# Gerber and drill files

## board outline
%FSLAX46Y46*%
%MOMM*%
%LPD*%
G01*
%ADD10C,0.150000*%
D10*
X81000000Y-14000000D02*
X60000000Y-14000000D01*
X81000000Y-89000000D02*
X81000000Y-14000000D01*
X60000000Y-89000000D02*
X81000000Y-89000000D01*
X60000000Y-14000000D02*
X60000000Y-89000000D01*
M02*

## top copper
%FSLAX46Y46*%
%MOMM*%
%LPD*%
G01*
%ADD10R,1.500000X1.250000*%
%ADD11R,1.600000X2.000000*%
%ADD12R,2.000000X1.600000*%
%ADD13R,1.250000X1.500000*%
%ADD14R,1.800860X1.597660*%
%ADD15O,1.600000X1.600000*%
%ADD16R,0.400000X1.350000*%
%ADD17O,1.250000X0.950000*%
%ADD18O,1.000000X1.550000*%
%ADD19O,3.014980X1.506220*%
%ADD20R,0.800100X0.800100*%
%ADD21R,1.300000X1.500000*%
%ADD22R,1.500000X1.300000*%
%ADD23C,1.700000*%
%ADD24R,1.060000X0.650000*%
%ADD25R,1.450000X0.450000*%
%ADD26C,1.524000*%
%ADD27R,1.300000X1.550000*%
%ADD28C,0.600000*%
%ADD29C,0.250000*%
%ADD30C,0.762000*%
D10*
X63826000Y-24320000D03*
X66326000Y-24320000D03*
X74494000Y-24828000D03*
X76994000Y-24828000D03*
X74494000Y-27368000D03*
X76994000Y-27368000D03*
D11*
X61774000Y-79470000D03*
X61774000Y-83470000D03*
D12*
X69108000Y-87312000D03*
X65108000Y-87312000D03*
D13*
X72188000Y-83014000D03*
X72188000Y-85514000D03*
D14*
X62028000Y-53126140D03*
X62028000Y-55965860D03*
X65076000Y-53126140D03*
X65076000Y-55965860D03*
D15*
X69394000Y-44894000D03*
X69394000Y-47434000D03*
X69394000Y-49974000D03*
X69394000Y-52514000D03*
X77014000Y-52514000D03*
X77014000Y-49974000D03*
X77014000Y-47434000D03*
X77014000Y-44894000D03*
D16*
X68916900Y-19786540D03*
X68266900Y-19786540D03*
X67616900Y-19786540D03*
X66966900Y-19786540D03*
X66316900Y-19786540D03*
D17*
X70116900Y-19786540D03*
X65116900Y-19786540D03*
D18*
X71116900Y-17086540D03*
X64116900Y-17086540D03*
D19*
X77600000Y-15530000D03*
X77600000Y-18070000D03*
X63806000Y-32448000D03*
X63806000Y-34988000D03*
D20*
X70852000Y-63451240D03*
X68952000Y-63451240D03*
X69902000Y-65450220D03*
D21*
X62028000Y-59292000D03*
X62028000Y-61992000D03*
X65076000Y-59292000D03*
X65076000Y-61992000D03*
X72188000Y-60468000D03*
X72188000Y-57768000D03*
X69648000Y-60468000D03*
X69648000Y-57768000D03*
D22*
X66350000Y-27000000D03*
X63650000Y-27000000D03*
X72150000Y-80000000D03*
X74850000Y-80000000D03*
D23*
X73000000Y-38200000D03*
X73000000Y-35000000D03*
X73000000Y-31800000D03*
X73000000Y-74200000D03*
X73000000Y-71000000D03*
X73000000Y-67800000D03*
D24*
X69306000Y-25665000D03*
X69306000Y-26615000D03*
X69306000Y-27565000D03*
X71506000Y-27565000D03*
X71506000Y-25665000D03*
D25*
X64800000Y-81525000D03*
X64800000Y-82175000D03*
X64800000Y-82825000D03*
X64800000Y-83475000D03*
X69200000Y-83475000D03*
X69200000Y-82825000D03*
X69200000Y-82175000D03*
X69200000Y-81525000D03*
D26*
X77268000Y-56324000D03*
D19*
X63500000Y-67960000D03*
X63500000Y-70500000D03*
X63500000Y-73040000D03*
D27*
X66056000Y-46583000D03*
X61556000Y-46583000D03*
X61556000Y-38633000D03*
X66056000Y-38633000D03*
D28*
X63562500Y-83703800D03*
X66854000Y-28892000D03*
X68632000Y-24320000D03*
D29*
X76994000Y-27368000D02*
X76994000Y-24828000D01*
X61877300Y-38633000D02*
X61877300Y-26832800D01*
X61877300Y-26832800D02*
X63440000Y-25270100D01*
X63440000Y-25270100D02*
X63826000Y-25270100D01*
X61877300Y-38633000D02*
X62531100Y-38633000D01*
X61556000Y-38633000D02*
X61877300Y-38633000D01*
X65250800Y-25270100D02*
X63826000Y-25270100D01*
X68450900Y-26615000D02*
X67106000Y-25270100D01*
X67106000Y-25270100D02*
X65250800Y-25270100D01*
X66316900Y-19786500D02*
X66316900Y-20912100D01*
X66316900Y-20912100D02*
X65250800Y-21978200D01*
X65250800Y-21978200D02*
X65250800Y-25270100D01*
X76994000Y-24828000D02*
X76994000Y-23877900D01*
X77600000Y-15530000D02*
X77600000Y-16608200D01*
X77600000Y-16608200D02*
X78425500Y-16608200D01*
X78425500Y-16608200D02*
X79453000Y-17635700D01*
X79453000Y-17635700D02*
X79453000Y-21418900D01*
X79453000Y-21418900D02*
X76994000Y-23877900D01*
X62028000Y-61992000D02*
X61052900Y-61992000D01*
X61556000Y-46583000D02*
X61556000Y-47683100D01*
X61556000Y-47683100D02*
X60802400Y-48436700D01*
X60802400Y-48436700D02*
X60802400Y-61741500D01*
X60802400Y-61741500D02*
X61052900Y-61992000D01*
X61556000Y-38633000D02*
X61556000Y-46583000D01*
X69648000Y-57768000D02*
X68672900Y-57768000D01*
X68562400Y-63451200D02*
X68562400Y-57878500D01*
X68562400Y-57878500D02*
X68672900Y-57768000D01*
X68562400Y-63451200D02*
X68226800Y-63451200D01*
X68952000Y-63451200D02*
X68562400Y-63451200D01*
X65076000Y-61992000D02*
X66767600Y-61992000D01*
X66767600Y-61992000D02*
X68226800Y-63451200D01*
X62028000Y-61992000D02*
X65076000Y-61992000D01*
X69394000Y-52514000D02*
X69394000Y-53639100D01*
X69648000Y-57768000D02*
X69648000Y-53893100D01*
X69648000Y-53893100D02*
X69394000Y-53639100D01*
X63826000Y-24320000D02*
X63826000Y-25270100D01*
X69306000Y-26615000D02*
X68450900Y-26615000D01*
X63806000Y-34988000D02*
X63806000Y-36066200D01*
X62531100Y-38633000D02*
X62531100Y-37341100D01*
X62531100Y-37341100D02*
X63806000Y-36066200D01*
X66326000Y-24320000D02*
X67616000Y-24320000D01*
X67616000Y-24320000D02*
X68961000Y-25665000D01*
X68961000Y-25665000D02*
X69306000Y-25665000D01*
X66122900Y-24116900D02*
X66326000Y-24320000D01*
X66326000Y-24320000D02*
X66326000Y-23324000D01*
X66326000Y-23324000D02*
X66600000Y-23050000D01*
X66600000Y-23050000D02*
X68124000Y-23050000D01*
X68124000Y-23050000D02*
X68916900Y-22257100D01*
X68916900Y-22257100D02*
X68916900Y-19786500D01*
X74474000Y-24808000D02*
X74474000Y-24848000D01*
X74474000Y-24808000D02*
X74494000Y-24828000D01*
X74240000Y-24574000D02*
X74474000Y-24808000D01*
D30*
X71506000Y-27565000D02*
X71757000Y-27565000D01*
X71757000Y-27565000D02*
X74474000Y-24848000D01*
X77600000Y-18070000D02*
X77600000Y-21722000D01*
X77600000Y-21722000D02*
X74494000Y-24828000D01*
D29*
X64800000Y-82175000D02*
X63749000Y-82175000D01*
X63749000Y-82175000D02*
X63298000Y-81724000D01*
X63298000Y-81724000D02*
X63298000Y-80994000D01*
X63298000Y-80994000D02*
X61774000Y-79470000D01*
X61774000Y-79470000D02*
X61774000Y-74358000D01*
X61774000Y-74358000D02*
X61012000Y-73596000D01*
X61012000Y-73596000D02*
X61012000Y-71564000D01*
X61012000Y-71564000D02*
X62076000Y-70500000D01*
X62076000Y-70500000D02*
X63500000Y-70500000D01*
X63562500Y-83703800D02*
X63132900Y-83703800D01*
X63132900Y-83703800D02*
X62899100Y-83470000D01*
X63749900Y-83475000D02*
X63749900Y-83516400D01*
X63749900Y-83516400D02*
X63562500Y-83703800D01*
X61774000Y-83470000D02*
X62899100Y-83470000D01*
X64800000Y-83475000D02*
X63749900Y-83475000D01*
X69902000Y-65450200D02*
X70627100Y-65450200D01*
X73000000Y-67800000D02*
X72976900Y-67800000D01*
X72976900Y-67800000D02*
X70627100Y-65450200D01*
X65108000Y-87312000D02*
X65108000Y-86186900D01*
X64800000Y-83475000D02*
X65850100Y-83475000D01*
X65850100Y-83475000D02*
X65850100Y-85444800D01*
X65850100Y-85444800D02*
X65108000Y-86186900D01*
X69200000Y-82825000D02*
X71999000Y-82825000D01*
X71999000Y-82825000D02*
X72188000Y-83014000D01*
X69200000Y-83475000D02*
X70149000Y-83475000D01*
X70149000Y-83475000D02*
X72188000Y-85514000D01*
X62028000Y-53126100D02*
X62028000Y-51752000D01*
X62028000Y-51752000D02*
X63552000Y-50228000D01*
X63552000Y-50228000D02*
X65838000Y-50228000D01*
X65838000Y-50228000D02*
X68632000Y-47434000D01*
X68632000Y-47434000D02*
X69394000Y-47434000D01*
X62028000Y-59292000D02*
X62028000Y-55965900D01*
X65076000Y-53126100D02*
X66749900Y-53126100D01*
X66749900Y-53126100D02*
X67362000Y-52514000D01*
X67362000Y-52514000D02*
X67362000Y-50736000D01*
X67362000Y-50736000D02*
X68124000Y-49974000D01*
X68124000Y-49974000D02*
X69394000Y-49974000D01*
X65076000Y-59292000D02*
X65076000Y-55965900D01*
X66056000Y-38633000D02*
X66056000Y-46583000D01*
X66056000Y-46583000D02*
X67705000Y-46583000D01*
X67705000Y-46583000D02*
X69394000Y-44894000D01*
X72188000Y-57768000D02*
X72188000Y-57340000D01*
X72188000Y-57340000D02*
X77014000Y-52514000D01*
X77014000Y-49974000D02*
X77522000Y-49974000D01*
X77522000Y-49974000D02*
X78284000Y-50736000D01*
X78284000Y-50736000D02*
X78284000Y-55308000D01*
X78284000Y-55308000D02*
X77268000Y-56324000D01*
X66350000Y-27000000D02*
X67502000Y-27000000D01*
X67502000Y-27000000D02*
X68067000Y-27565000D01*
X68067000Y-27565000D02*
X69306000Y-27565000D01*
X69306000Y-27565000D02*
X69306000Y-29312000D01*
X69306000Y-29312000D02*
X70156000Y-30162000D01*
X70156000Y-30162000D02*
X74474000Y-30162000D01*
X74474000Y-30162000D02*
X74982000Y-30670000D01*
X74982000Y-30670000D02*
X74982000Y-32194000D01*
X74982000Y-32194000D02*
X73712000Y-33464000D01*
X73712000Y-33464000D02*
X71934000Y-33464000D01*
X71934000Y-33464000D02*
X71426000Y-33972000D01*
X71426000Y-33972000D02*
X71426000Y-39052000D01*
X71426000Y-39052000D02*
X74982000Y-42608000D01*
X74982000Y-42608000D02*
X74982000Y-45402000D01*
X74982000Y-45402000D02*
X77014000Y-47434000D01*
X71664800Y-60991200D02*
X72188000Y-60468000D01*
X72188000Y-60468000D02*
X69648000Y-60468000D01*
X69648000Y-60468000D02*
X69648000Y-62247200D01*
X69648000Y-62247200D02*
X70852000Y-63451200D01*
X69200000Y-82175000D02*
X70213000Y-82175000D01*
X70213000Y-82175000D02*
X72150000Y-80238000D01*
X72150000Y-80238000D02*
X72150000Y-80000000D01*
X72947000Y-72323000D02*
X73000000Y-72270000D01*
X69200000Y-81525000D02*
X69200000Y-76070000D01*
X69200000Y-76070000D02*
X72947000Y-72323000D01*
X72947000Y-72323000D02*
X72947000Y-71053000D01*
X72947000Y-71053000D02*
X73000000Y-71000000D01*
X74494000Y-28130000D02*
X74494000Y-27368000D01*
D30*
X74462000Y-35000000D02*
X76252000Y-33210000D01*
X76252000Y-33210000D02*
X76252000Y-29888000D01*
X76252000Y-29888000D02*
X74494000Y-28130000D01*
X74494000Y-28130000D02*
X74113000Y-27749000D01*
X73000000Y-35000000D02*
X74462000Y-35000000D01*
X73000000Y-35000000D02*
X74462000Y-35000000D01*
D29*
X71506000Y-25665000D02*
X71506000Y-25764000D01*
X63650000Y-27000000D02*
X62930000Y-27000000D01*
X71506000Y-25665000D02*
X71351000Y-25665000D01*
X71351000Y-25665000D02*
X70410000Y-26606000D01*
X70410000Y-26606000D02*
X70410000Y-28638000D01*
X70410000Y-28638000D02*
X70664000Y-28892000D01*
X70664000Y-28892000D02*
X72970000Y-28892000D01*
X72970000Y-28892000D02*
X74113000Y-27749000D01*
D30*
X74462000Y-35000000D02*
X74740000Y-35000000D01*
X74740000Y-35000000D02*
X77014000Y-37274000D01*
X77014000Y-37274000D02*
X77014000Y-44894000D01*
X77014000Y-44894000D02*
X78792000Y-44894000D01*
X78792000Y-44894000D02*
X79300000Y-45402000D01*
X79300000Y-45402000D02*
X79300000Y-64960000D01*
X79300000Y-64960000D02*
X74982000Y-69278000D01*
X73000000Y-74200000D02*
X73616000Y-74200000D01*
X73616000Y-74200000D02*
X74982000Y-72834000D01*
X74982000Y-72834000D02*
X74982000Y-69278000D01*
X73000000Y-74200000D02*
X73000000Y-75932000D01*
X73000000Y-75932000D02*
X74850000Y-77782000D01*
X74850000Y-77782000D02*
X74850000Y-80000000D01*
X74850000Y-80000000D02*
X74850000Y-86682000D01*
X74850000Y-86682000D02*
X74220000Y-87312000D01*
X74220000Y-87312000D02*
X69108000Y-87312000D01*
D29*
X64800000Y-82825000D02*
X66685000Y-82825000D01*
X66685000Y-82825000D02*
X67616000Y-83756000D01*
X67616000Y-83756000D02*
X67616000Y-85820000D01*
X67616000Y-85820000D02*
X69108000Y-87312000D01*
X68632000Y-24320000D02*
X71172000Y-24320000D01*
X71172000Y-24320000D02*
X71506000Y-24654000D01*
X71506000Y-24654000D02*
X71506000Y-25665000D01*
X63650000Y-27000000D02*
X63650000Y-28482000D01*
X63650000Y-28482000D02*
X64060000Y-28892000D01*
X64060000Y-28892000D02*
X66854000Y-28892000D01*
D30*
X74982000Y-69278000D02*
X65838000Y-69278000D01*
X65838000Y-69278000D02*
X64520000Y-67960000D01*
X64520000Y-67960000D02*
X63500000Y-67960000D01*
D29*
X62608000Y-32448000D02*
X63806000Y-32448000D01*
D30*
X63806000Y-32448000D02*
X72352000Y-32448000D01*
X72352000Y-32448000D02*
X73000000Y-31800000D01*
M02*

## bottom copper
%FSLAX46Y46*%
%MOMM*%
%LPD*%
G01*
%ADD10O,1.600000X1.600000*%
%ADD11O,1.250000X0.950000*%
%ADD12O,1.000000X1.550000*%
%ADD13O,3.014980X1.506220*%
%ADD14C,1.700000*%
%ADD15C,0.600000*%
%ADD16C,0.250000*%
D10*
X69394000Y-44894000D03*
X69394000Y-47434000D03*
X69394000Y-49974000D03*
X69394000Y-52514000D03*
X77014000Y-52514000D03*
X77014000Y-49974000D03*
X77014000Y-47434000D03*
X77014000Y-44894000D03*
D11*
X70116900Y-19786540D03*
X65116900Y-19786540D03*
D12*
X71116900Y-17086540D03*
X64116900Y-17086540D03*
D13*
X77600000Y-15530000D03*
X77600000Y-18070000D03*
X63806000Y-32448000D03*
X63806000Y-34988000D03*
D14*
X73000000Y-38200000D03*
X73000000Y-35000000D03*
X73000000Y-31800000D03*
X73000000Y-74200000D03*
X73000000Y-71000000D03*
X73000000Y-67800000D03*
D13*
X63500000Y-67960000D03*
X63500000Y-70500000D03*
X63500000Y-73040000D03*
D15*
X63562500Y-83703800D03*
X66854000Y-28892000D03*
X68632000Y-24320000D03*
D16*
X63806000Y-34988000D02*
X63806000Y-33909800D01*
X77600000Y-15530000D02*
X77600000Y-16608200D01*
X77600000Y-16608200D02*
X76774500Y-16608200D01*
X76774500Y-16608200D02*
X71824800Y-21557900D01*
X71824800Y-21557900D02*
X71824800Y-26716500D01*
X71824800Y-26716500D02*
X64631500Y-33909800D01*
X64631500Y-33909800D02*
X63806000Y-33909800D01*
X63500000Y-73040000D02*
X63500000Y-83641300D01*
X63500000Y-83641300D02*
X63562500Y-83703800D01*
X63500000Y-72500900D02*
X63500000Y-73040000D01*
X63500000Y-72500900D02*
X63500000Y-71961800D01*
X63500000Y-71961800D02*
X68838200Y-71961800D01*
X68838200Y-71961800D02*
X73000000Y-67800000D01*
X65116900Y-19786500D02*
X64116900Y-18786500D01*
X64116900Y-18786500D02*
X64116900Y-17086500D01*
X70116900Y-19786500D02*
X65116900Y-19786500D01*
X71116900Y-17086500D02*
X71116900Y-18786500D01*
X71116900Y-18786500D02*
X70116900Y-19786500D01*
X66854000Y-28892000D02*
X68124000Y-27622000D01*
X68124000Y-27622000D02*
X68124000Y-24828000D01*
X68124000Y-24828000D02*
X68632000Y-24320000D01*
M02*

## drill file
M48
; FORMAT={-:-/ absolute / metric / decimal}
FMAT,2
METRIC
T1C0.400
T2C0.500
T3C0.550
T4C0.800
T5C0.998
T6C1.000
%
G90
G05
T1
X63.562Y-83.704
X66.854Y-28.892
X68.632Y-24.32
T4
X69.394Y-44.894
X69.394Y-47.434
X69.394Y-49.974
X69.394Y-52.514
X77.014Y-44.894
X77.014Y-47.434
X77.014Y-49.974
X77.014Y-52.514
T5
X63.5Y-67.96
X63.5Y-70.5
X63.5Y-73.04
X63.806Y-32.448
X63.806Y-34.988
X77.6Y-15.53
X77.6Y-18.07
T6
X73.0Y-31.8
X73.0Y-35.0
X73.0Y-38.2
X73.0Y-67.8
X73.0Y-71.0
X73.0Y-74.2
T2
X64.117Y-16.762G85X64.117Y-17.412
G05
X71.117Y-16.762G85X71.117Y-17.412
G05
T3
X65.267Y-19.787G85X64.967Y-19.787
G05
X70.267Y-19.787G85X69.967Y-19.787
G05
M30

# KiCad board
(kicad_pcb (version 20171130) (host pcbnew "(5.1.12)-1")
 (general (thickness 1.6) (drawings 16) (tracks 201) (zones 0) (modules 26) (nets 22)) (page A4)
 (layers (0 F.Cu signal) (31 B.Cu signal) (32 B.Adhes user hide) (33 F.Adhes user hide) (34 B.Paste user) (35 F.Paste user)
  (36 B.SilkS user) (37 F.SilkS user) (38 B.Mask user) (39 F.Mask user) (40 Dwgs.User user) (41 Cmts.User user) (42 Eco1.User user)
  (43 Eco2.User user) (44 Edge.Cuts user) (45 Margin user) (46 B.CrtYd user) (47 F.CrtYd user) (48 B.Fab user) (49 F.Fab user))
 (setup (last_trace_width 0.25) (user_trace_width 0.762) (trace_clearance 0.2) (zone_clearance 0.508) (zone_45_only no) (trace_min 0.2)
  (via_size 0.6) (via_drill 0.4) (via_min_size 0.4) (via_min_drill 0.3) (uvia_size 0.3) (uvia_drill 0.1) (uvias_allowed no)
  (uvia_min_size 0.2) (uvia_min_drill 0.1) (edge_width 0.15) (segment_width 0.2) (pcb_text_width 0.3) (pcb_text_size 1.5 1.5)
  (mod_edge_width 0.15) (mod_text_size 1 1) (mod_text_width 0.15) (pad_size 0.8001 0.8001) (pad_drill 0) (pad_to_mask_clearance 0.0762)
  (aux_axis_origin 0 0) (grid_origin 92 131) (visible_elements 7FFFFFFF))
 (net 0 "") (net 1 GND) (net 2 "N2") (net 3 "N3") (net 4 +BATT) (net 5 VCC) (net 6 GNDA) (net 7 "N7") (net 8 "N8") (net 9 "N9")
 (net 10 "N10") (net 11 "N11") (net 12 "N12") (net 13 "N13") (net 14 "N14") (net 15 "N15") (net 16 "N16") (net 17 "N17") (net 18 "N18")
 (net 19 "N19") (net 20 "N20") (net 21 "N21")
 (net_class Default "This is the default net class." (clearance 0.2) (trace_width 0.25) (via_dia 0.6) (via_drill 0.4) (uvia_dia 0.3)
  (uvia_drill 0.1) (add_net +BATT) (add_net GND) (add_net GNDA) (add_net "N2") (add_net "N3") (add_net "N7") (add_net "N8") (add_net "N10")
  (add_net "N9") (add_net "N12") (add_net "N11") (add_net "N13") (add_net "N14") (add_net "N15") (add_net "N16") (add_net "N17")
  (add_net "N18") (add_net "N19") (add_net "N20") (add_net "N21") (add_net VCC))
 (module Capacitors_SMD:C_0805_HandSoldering (layer F.Cu) (at 65.076 24.32)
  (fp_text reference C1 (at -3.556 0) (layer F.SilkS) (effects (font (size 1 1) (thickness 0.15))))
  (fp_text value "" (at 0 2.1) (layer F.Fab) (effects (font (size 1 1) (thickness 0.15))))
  (pad 1 smd rect (at -1.25 0) (size 1.5 1.25) (layers F.Cu F.Paste F.Mask) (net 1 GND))
  (pad 2 smd rect (at 1.25 0) (size 1.5 1.25) (layers F.Cu F.Paste F.Mask) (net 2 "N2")))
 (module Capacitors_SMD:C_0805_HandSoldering (layer F.Cu) (at 75.744 24.828)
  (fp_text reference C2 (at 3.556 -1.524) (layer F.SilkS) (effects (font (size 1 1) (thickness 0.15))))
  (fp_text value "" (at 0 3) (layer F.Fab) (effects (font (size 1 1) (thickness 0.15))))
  (pad 1 smd rect (at -1.25 0) (size 1.5 1.25) (layers F.Cu F.Paste F.Mask) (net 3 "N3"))
  (pad 2 smd rect (at 1.25 0) (size 1.5 1.25) (layers F.Cu F.Paste F.Mask) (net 1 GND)))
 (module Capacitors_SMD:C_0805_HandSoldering (layer F.Cu) (at 75.744 27.368)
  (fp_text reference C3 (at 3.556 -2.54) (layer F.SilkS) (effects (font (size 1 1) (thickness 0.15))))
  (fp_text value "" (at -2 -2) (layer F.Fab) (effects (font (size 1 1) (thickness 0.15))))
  (pad 1 smd rect (at -1.25 0) (size 1.5 1.25) (layers F.Cu F.Paste F.Mask) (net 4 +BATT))
  (pad 2 smd rect (at 1.25 0) (size 1.5 1.25) (layers F.Cu F.Paste F.Mask) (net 1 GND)))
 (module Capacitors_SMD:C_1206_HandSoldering (layer F.Cu) (at 61.774 81.47 270)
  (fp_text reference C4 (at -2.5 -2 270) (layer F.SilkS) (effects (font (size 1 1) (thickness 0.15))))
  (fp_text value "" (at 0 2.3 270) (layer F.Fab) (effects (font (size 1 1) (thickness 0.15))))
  (pad 1 smd rect (at -2 0 270) (size 2 1.6) (layers F.Cu F.Paste F.Mask) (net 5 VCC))
  (pad 2 smd rect (at 2 0 270) (size 2 1.6) (layers F.Cu F.Paste F.Mask) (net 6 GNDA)))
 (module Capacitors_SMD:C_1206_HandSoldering (layer F.Cu) (at 67.108 87.312 180)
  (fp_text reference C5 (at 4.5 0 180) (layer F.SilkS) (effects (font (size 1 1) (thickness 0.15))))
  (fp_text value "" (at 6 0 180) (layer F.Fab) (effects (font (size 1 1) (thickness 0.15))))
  (pad 1 smd rect (at -2 0 180) (size 2 1.6) (layers F.Cu F.Paste F.Mask) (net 4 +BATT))
  (pad 2 smd rect (at 2 0 180) (size 2 1.6) (layers F.Cu F.Paste F.Mask) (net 6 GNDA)))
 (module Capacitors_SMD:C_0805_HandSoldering (layer F.Cu) (at 72.188 84.264 270)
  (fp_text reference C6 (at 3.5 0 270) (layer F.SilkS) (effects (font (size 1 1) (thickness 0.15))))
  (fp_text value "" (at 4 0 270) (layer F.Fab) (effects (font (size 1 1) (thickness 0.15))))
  (pad 1 smd rect (at -1.25 0 270) (size 1.5 1.25) (layers F.Cu F.Paste F.Mask) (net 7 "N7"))
  (pad 2 smd rect (at 1.25 0 270) (size 1.5 1.25) (layers F.Cu F.Paste F.Mask) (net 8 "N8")))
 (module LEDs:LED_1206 (layer F.Cu) (at 62.028 54.546 90)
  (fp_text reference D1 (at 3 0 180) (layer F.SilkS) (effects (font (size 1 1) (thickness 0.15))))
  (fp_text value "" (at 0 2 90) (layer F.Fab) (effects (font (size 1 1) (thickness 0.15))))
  (pad 2 smd rect (at 1.41986 0 270) (size 1.59766 1.80086) (layers F.Cu F.Paste F.Mask) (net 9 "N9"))
  (pad 1 smd rect (at -1.41986 0 270) (size 1.59766 1.80086) (layers F.Cu F.Paste F.Mask) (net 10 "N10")))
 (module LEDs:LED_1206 (layer F.Cu) (at 65.076 54.546 90)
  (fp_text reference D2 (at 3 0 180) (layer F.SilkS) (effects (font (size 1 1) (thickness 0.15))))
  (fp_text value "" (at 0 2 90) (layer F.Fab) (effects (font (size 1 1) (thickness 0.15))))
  (pad 2 smd rect (at 1.41986 0 270) (size 1.59766 1.80086) (layers F.Cu F.Paste F.Mask) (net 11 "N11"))
  (pad 1 smd rect (at -1.41986 0 270) (size 1.59766 1.80086) (layers F.Cu F.Paste F.Mask) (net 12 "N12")))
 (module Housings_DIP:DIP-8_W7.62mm (layer F.Cu) (at 69.394 44.894)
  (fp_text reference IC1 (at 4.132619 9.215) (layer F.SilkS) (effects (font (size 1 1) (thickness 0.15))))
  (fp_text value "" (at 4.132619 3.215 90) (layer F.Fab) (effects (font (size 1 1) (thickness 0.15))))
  (pad 1 thru_hole oval (at 0 0) (size 1.6 1.6) (drill 0.8) (layers *.Cu *.Mask F.SilkS) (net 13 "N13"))
  (pad 2 thru_hole oval (at 0 2.54) (size 1.6 1.6) (drill 0.8) (layers *.Cu *.Mask F.SilkS) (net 9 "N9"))
  (pad 3 thru_hole oval (at 0 5.08) (size 1.6 1.6) (drill 0.8) (layers *.Cu *.Mask F.SilkS) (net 11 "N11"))
  (pad 4 thru_hole oval (at 0 7.62) (size 1.6 1.6) (drill 0.8) (layers *.Cu *.Mask F.SilkS) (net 1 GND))
  (pad 5 thru_hole oval (at 7.62 7.62) (size 1.6 1.6) (drill 0.8) (layers *.Cu *.Mask F.SilkS) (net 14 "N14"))
  (pad 6 thru_hole oval (at 7.62 5.08) (size 1.6 1.6) (drill 0.8) (layers *.Cu *.Mask F.SilkS) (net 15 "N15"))
  (pad 7 thru_hole oval (at 7.62 2.54) (size 1.6 1.6) (drill 0.8) (layers *.Cu *.Mask F.SilkS) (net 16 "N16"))
  (pad 8 thru_hole oval (at 7.62 0) (size 1.6 1.6) (drill 0.8) (layers *.Cu *.Mask F.SilkS) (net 4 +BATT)))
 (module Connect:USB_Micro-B (layer F.Cu) (at 67.616 18.224 180)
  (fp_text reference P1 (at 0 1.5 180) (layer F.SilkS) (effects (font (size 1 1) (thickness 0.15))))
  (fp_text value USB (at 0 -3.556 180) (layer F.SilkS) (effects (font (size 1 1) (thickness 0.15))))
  (pad 1 smd rect (at -1.3009 -1.56254 270) (size 1.35 0.4) (layers F.Cu F.Paste F.Mask) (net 2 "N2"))
  (pad 2 smd rect (at -0.6509 -1.56254 270) (size 1.35 0.4) (layers F.Cu F.Paste F.Mask))
  (pad 3 smd rect (at -0.0009 -1.56254 270) (size 1.35 0.4) (layers F.Cu F.Paste F.Mask))
  (pad 4 smd rect (at 0.6491 -1.56254 270) (size 1.35 0.4) (layers F.Cu F.Paste F.Mask))
  (pad 5 smd rect (at 1.2991 -1.56254 270) (size 1.35 0.4) (layers F.Cu F.Paste F.Mask) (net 1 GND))
  (pad 6 thru_hole oval (at -2.5009 -1.56254 270) (size 0.95 1.25) (drill oval 0.55 0.85) (layers *.Cu *.Mask F.SilkS) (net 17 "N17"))
  (pad 6 thru_hole oval (at 2.4991 -1.56254 270) (size 0.95 1.25) (drill oval 0.55 0.85) (layers *.Cu *.Mask F.SilkS) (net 17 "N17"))
  (pad 6 thru_hole oval (at -3.5009 1.13746 270) (size 1.55 1) (drill oval 1.15 0.5) (layers *.Cu *.Mask F.SilkS) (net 17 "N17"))
  (pad 6 thru_hole oval (at 3.4991 1.13746 270) (size 1.55 1) (drill oval 1.15 0.5) (layers *.Cu *.Mask F.SilkS) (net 17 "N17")))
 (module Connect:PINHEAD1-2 (layer F.Cu) (at 77.6 16.8 270)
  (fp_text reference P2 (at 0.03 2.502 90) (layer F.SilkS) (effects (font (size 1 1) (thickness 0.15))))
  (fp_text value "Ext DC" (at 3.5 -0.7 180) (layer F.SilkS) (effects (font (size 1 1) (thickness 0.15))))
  (pad 1 thru_hole oval (at -1.27 0 270) (size 1.50622 3.01498) (drill 0.99822) (layers *.Cu *.Mask) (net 1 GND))
  (pad 2 thru_hole oval (at 1.27 0 270) (size 1.50622 3.01498) (drill 0.99822) (layers *.Cu *.Mask) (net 3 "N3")))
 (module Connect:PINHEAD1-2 (layer F.Cu) (at 63.806 33.718 270)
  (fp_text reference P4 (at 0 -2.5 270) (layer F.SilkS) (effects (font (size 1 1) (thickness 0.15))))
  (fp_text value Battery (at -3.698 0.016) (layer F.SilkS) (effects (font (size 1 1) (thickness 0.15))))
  (pad 1 thru_hole oval (at -1.27 0 270) (size 1.50622 3.01498) (drill 0.99822) (layers *.Cu *.Mask) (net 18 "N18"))
  (pad 2 thru_hole oval (at 1.27 0 270) (size 1.50622 3.01498) (drill 0.99822) (layers *.Cu *.Mask) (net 1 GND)))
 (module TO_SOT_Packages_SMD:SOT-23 (layer F.Cu) (at 69.902 64.452 180)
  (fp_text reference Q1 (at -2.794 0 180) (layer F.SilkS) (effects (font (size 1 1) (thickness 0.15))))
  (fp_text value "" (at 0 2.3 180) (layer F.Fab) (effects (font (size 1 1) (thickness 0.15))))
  (pad 2 smd rect (at -0.95 1.00076 180) (size 0.8001 0.8001) (layers F.Cu F.Paste F.Mask) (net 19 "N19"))
  (pad 3 smd rect (at 0.95 1.00076 180) (size 0.8001 0.8001) (layers F.Cu F.Paste F.Mask) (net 1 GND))
  (pad 1 smd rect (at 0 -0.99822 180) (size 0.8001 0.8001) (layers F.Cu F.Paste F.Mask) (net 6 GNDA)))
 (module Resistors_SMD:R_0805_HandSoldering (layer F.Cu) (at 62.028 60.642 270)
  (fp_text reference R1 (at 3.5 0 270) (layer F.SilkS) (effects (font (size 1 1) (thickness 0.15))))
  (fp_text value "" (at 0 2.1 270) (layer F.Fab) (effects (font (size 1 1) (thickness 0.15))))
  (pad 1 smd rect (at -1.35 0 270) (size 1.5 1.3) (layers F.Cu F.Paste F.Mask) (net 10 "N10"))
  (pad 2 smd rect (at 1.35 0 270) (size 1.5 1.3) (layers F.Cu F.Paste F.Mask) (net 1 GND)))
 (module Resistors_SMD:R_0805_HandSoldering (layer F.Cu) (at 65.076 60.642 270)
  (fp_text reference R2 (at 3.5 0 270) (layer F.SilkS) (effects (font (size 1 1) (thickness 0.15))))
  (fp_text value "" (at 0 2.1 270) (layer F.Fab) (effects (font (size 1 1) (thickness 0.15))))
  (pad 1 smd rect (at -1.35 0 270) (size 1.5 1.3) (layers F.Cu F.Paste F.Mask) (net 12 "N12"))
  (pad 2 smd rect (at 1.35 0 270) (size 1.5 1.3) (layers F.Cu F.Paste F.Mask) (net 1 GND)))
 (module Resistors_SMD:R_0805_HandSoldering (layer F.Cu) (at 72.188 59.118 90)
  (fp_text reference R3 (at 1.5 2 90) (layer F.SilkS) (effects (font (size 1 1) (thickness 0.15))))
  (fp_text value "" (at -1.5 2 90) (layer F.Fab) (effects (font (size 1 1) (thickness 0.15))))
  (pad 1 smd rect (at -1.35 0 90) (size 1.5 1.3) (layers F.Cu F.Paste F.Mask) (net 19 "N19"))
  (pad 2 smd rect (at 1.35 0 90) (size 1.5 1.3) (layers F.Cu F.Paste F.Mask) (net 14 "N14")))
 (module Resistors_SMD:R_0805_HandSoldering (layer F.Cu) (at 69.648 59.118 90)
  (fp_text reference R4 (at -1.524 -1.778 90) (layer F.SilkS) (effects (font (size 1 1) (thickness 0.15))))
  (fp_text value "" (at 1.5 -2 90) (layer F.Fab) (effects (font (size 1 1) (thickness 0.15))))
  (pad 1 smd rect (at -1.35 0 90) (size 1.5 1.3) (layers F.Cu F.Paste F.Mask) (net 19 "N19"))
  (pad 2 smd rect (at 1.35 0 90) (size 1.5 1.3) (layers F.Cu F.Paste F.Mask) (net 1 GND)))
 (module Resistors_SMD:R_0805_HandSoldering (layer F.Cu) (at 65 27 180)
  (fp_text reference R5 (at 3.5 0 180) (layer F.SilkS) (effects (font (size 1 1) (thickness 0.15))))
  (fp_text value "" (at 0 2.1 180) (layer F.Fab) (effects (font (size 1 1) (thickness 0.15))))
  (pad 1 smd rect (at -1.35 0 180) (size 1.5 1.3) (layers F.Cu F.Paste F.Mask) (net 16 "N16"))
  (pad 2 smd rect (at 1.35 0 180) (size 1.5 1.3) (layers F.Cu F.Paste F.Mask) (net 4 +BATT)))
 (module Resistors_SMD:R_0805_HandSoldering (layer F.Cu) (at 73.5 80)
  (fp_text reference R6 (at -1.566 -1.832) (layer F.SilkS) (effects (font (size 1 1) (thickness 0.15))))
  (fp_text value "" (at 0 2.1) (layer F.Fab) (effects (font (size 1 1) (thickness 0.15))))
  (pad 1 smd rect (at -1.35 0) (size 1.5 1.3) (layers F.Cu F.Paste F.Mask) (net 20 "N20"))
  (pad 2 smd rect (at 1.35 0) (size 1.5 1.3) (layers F.Cu F.Paste F.Mask) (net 4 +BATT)))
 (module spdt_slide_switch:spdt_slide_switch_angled (layer F.Cu) (at 73 35 90)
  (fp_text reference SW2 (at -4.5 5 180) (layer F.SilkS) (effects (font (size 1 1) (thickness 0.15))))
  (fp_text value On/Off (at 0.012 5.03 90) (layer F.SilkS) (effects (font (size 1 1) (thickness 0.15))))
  (pad 1 thru_hole circle (at -3.2 0 90) (size 1.7 1.7) (drill 1) (layers *.Cu *.Mask F.SilkS))
  (pad 2 thru_hole circle (at 0 0 90) (size 1.7 1.7) (drill 1) (layers *.Cu *.Mask F.SilkS) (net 4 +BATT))
  (pad 3 thru_hole circle (at 3.2 0 90) (size 1.7 1.7) (drill 1) (layers *.Cu *.Mask F.SilkS) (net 18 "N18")))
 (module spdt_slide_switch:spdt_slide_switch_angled (layer F.Cu) (at 73 71 90)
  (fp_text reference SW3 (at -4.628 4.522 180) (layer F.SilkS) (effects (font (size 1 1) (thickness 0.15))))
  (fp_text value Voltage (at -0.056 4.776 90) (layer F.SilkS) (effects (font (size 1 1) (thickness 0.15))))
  (pad 1 thru_hole circle (at -3.2 0 90) (size 1.7 1.7) (drill 1) (layers *.Cu *.Mask F.SilkS) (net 4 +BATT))
  (pad 2 thru_hole circle (at 0 0 90) (size 1.7 1.7) (drill 1) (layers *.Cu *.Mask F.SilkS) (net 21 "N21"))
  (pad 3 thru_hole circle (at 3.2 0 90) (size 1.7 1.7) (drill 1) (layers *.Cu *.Mask F.SilkS) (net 6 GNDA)))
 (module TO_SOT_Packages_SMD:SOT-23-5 (layer F.Cu) (at 70.406 26.615)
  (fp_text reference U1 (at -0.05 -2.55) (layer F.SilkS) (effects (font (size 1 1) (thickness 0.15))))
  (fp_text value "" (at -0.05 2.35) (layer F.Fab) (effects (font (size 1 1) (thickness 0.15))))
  (pad 1 smd rect (at -1.1 -0.95) (size 1.06 0.65) (layers F.Cu F.Paste F.Mask) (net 2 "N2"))
  (pad 2 smd rect (at -1.1 0) (size 1.06 0.65) (layers F.Cu F.Paste F.Mask) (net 1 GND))
  (pad 3 smd rect (at -1.1 0.95) (size 1.06 0.65) (layers F.Cu F.Paste F.Mask) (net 16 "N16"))
  (pad 4 smd rect (at 1.1 0.95) (size 1.06 0.65) (layers F.Cu F.Paste F.Mask) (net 3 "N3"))
  (pad 5 smd rect (at 1.1 -0.95) (size 1.06 0.65) (layers F.Cu F.Paste F.Mask) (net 4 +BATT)))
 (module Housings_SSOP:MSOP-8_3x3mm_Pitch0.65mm (layer F.Cu) (at 67 82.5)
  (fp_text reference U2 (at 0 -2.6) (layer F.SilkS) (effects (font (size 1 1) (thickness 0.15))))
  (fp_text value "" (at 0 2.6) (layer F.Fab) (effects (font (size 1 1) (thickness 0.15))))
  (pad 1 smd rect (at -2.2 -0.975) (size 1.45 0.45) (layers F.Cu F.Paste F.Mask))
  (pad 2 smd rect (at -2.2 -0.325) (size 1.45 0.45) (layers F.Cu F.Paste F.Mask) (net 5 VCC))
  (pad 3 smd rect (at -2.2 0.325) (size 1.45 0.45) (layers F.Cu F.Paste F.Mask) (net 4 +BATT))
  (pad 4 smd rect (at -2.2 0.975) (size 1.45 0.45) (layers F.Cu F.Paste F.Mask) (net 6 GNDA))
  (pad 5 smd rect (at 2.2 0.975) (size 1.45 0.45) (layers F.Cu F.Paste F.Mask) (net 8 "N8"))
  (pad 6 smd rect (at 2.2 0.325) (size 1.45 0.45) (layers F.Cu F.Paste F.Mask) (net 7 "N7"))
  (pad 7 smd rect (at 2.2 -0.325) (size 1.45 0.45) (layers F.Cu F.Paste F.Mask) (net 20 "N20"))
  (pad 8 smd rect (at 2.2 -0.975) (size 1.45 0.45) (layers F.Cu F.Paste F.Mask) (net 21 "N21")))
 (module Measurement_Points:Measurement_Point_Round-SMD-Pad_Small (layer F.Cu) (at 77.268 56.324)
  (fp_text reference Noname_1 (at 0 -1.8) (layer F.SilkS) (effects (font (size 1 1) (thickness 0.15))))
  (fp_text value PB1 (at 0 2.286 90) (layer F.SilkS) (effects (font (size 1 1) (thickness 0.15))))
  (pad 1 smd circle (at 0 0) (size 1.524 1.524) (layers F.Cu F.Paste F.Mask) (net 15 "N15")))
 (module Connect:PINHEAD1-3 (layer F.Cu) (at 63.5 70.5 270)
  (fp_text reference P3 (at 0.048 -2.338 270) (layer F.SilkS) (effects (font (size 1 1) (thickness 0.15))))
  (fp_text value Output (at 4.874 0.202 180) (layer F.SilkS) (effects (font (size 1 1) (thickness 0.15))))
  (pad 1 thru_hole oval (at -2.54 0 270) (size 1.50622 3.01498) (drill 0.99822) (layers *.Cu *.Mask) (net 4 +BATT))
  (pad 2 thru_hole oval (at 0 0 270) (size 1.50622 3.01498) (drill 0.99822) (layers *.Cu *.Mask) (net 5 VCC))
  (pad 3 thru_hole oval (at 2.54 0 270) (size 1.50622 3.01498) (drill 0.99822) (layers *.Cu *.Mask) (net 6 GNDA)))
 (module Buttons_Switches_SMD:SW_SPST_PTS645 (layer F.Cu) (at 63.806 42.608 90)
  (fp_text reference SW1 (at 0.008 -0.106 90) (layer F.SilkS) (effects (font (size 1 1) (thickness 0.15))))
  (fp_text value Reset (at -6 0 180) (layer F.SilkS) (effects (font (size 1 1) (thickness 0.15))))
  (pad 2 smd rect (at -3.975 2.25 90) (size 1.55 1.3) (layers F.Cu F.Paste F.Mask) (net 13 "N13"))
  (pad 1 smd rect (at -3.975 -2.25 90) (size 1.55 1.3) (layers F.Cu F.Paste F.Mask) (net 1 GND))
  (pad 1 smd rect (at 3.975 -2.25 90) (size 1.55 1.3) (layers F.Cu F.Paste F.Mask) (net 1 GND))
  (pad 2 smd rect (at 3.975 2.25 90) (size 1.55 1.3) (layers F.Cu F.Paste F.Mask) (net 13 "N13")))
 (gr_line (start 81 14) (end 60 14) (angle 90) (layer Edge.Cuts) (width 0.15))
 (gr_line (start 81 89) (end 81 14) (angle 90) (layer Edge.Cuts) (width 0.15))
 (gr_line (start 60 89) (end 81 89) (angle 90) (layer Edge.Cuts) (width 0.15))
 (gr_line (start 60 14) (end 60 89) (angle 90) (layer Edge.Cuts) (width 0.15))
 (segment (start 63.806 34.988) (end 63.806 33.9098) (width 0.25) (layer B.Cu) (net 1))
 (segment (start 77.6 15.53) (end 77.6 16.6082) (width 0.25) (layer B.Cu) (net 1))
 (segment (start 77.6 16.6082) (end 76.7745 16.6082) (width 0.25) (layer B.Cu) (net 1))
 (segment (start 76.7745 16.6082) (end 71.8248 21.5579) (width 0.25) (layer B.Cu) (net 1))
 (segment (start 71.8248 21.5579) (end 71.8248 26.7165) (width 0.25) (layer B.Cu) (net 1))
 (segment (start 71.8248 26.7165) (end 64.6315 33.9098) (width 0.25) (layer B.Cu) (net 1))
 (segment (start 64.6315 33.9098) (end 63.806 33.9098) (width 0.25) (layer B.Cu) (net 1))
 (segment (start 76.994 27.368) (end 76.994 24.828) (width 0.25) (layer F.Cu) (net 1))
 (segment (start 61.8773 38.633) (end 61.8773 26.8328) (width 0.25) (layer F.Cu) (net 1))
 (segment (start 61.8773 26.8328) (end 63.44 25.2701) (width 0.25) (layer F.Cu) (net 1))
 (segment (start 63.44 25.2701) (end 63.826 25.2701) (width 0.25) (layer F.Cu) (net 1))
 (segment (start 61.8773 38.633) (end 62.5311 38.633) (width 0.25) (layer F.Cu) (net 1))
 (segment (start 61.556 38.633) (end 61.8773 38.633) (width 0.25) (layer F.Cu) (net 1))
 (segment (start 65.2508 25.2701) (end 63.826 25.2701) (width 0.25) (layer F.Cu) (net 1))
 (segment (start 68.4509 26.615) (end 67.106 25.2701) (width 0.25) (layer F.Cu) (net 1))
 (segment (start 67.106 25.2701) (end 65.2508 25.2701) (width 0.25) (layer F.Cu) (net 1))
 (segment (start 66.3169 19.7865) (end 66.3169 20.9121) (width 0.25) (layer F.Cu) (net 1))
 (segment (start 66.3169 20.9121) (end 65.2508 21.9782) (width 0.25) (layer F.Cu) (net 1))
 (segment (start 65.2508 21.9782) (end 65.2508 25.2701) (width 0.25) (layer F.Cu) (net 1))
 (segment (start 76.994 24.828) (end 76.994 23.8779) (width 0.25) (layer F.Cu) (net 1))
 (segment (start 77.6 15.53) (end 77.6 16.6082) (width 0.25) (layer F.Cu) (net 1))
 (segment (start 77.6 16.6082) (end 78.4255 16.6082) (width 0.25) (layer F.Cu) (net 1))
 (segment (start 78.4255 16.6082) (end 79.453 17.6357) (width 0.25) (layer F.Cu) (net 1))
 (segment (start 79.453 17.6357) (end 79.453 21.4189) (width 0.25) (layer F.Cu) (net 1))
 (segment (start 79.453 21.4189) (end 76.994 23.8779) (width 0.25) (layer F.Cu) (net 1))
 (segment (start 62.028 61.992) (end 61.0529 61.992) (width 0.25) (layer F.Cu) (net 1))
 (segment (start 61.556 46.583) (end 61.556 47.6831) (width 0.25) (layer F.Cu) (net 1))
 (segment (start 61.556 47.6831) (end 60.8024 48.4367) (width 0.25) (layer F.Cu) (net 1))
 (segment (start 60.8024 48.4367) (end 60.8024 61.7415) (width 0.25) (layer F.Cu) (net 1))
 (segment (start 60.8024 61.7415) (end 61.0529 61.992) (width 0.25) (layer F.Cu) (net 1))
 (segment (start 61.556 38.633) (end 61.556 46.583) (width 0.25) (layer F.Cu) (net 1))
 (segment (start 69.648 57.768) (end 68.6729 57.768) (width 0.25) (layer F.Cu) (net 1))
 (segment (start 68.5624 63.4512) (end 68.5624 57.8785) (width 0.25) (layer F.Cu) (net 1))
 (segment (start 68.5624 57.8785) (end 68.6729 57.768) (width 0.25) (layer F.Cu) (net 1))
 (segment (start 68.5624 63.4512) (end 68.2268 63.4512) (width 0.25) (layer F.Cu) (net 1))
 (segment (start 68.952 63.4512) (end 68.5624 63.4512) (width 0.25) (layer F.Cu) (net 1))
 (segment (start 65.076 61.992) (end 66.7676 61.992) (width 0.25) (layer F.Cu) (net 1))
 (segment (start 66.7676 61.992) (end 68.2268 63.4512) (width 0.25) (layer F.Cu) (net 1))
 (segment (start 62.028 61.992) (end 65.076 61.992) (width 0.25) (layer F.Cu) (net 1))
 (segment (start 69.394 52.514) (end 69.394 53.6391) (width 0.25) (layer F.Cu) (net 1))
 (segment (start 69.648 57.768) (end 69.648 53.8931) (width 0.25) (layer F.Cu) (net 1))
 (segment (start 69.648 53.8931) (end 69.394 53.6391) (width 0.25) (layer F.Cu) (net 1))
 (segment (start 63.826 24.32) (end 63.826 25.2701) (width 0.25) (layer F.Cu) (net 1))
 (segment (start 69.306 26.615) (end 68.4509 26.615) (width 0.25) (layer F.Cu) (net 1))
 (segment (start 63.806 34.988) (end 63.806 36.0662) (width 0.25) (layer F.Cu) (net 1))
 (segment (start 62.5311 38.633) (end 62.5311 37.3411) (width 0.25) (layer F.Cu) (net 1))
 (segment (start 62.5311 37.3411) (end 63.806 36.0662) (width 0.25) (layer F.Cu) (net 1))
 (segment (start 66.326 24.32) (end 67.616 24.32) (width 0.25) (layer F.Cu) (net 2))
 (segment (start 67.616 24.32) (end 68.961 25.665) (width 0.25) (layer F.Cu) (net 2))
 (segment (start 68.961 25.665) (end 69.306 25.665) (width 0.25) (layer F.Cu) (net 2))
 (segment (start 66.1229 24.1169) (end 66.326 24.32) (width 0.25) (layer F.Cu) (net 2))
 (segment (start 66.326 24.32) (end 66.326 23.324) (width 0.25) (layer F.Cu) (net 2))
 (segment (start 66.326 23.324) (end 66.6 23.05) (width 0.25) (layer F.Cu) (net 2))
 (segment (start 66.6 23.05) (end 68.124 23.05) (width 0.25) (layer F.Cu) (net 2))
 (segment (start 68.124 23.05) (end 68.9169 22.2571) (width 0.25) (layer F.Cu) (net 2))
 (segment (start 68.9169 22.2571) (end 68.9169 19.7865) (width 0.25) (layer F.Cu) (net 2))
 (segment (start 74.474 24.808) (end 74.474 24.848) (width 0.25) (layer F.Cu) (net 3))
 (segment (start 74.474 24.808) (end 74.494 24.828) (width 0.25) (layer F.Cu) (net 3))
 (segment (start 74.24 24.574) (end 74.474 24.808) (width 0.25) (layer F.Cu) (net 3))
 (segment (start 71.506 27.565) (end 71.757 27.565) (width 0.762) (layer F.Cu) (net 3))
 (segment (start 71.757 27.565) (end 74.474 24.848) (width 0.762) (layer F.Cu) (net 3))
 (segment (start 77.6 18.07) (end 77.6 21.722) (width 0.762) (layer F.Cu) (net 3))
 (segment (start 77.6 21.722) (end 74.494 24.828) (width 0.762) (layer F.Cu) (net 3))
 (segment (start 64.8 82.175) (end 63.749 82.175) (width 0.25) (layer F.Cu) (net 5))
 (segment (start 63.749 82.175) (end 63.298 81.724) (width 0.25) (layer F.Cu) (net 5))
 (segment (start 63.298 81.724) (end 63.298 80.994) (width 0.25) (layer F.Cu) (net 5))
 (segment (start 63.298 80.994) (end 61.774 79.47) (width 0.25) (layer F.Cu) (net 5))
 (segment (start 61.774 79.47) (end 61.774 74.358) (width 0.25) (layer F.Cu) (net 5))
 (segment (start 61.774 74.358) (end 61.012 73.596) (width 0.25) (layer F.Cu) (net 5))
 (segment (start 61.012 73.596) (end 61.012 71.564) (width 0.25) (layer F.Cu) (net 5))
 (segment (start 61.012 71.564) (end 62.076 70.5) (width 0.25) (layer F.Cu) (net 5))
 (segment (start 62.076 70.5) (end 63.5 70.5) (width 0.25) (layer F.Cu) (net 5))
 (segment (start 63.5 73.04) (end 63.5 83.6413) (width 0.25) (layer B.Cu) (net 6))
 (segment (start 63.5 83.6413) (end 63.5625 83.7038) (width 0.25) (layer B.Cu) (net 6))
 (segment (start 63.5625 83.7038) (end 63.1329 83.7038) (width 0.25) (layer F.Cu) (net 6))
 (segment (start 63.1329 83.7038) (end 62.8991 83.47) (width 0.25) (layer F.Cu) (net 6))
 (segment (start 63.7499 83.475) (end 63.7499 83.5164) (width 0.25) (layer F.Cu) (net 6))
 (segment (start 63.7499 83.5164) (end 63.5625 83.7038) (width 0.25) (layer F.Cu) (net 6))
 (segment (start 61.774 83.47) (end 62.8991 83.47) (width 0.25) (layer F.Cu) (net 6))
 (segment (start 64.8 83.475) (end 63.7499 83.475) (width 0.25) (layer F.Cu) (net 6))
 (segment (start 63.5 72.5009) (end 63.5 73.04) (width 0.25) (layer B.Cu) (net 6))
 (segment (start 63.5 72.5009) (end 63.5 71.9618) (width 0.25) (layer B.Cu) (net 6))
 (segment (start 69.902 65.4502) (end 70.6271 65.4502) (width 0.25) (layer F.Cu) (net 6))
 (segment (start 73 67.8) (end 72.9769 67.8) (width 0.25) (layer F.Cu) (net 6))
 (segment (start 72.9769 67.8) (end 70.6271 65.4502) (width 0.25) (layer F.Cu) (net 6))
 (segment (start 65.108 87.312) (end 65.108 86.1869) (width 0.25) (layer F.Cu) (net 6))
 (segment (start 64.8 83.475) (end 65.8501 83.475) (width 0.25) (layer F.Cu) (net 6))
 (segment (start 65.8501 83.475) (end 65.8501 85.4448) (width 0.25) (layer F.Cu) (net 6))
 (segment (start 65.8501 85.4448) (end 65.108 86.1869) (width 0.25) (layer F.Cu) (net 6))
 (segment (start 63.5 71.9618) (end 68.8382 71.9618) (width 0.25) (layer B.Cu) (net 6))
 (segment (start 68.8382 71.9618) (end 73 67.8) (width 0.25) (layer B.Cu) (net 6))
 (via (at 63.5625 83.7038) (size 0.6) (layers F.Cu B.Cu) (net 6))
 (segment (start 69.2 82.825) (end 71.999 82.825) (width 0.25) (layer F.Cu) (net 7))
 (segment (start 71.999 82.825) (end 72.188 83.014) (width 0.25) (layer F.Cu) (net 7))
 (segment (start 69.2 83.475) (end 70.149 83.475) (width 0.25) (layer F.Cu) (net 8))
 (segment (start 70.149 83.475) (end 72.188 85.514) (width 0.25) (layer F.Cu) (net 8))
 (segment (start 62.028 53.1261) (end 62.028 51.752) (width 0.25) (layer F.Cu) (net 9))
 (segment (start 62.028 51.752) (end 63.552 50.228) (width 0.25) (layer F.Cu) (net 9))
 (segment (start 63.552 50.228) (end 65.838 50.228) (width 0.25) (layer F.Cu) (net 9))
 (segment (start 65.838 50.228) (end 68.632 47.434) (width 0.25) (layer F.Cu) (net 9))
 (segment (start 68.632 47.434) (end 69.394 47.434) (width 0.25) (layer F.Cu) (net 9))
 (segment (start 62.028 59.292) (end 62.028 55.9659) (width 0.25) (layer F.Cu) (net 10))
 (segment (start 65.076 53.1261) (end 66.7499 53.1261) (width 0.25) (layer F.Cu) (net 11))
 (segment (start 66.7499 53.1261) (end 67.362 52.514) (width 0.25) (layer F.Cu) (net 11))
 (segment (start 67.362 52.514) (end 67.362 50.736) (width 0.25) (layer F.Cu) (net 11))
 (segment (start 67.362 50.736) (end 68.124 49.974) (width 0.25) (layer F.Cu) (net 11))
 (segment (start 68.124 49.974) (end 69.394 49.974) (width 0.25) (layer F.Cu) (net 11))
 (segment (start 65.076 59.292) (end 65.076 55.9659) (width 0.25) (layer F.Cu) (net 12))
 (segment (start 66.056 38.633) (end 66.056 46.583) (width 0.25) (layer F.Cu) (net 13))
 (segment (start 66.056 46.583) (end 67.705 46.583) (width 0.25) (layer F.Cu) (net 13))
 (segment (start 67.705 46.583) (end 69.394 44.894) (width 0.25) (layer F.Cu) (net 13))
 (segment (start 72.188 57.768) (end 72.188 57.34) (width 0.25) (layer F.Cu) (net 14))
 (segment (start 72.188 57.34) (end 77.014 52.514) (width 0.25) (layer F.Cu) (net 14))
 (segment (start 77.014 49.974) (end 77.522 49.974) (width 0.25) (layer F.Cu) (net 15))
 (segment (start 77.522 49.974) (end 78.284 50.736) (width 0.25) (layer F.Cu) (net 15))
 (segment (start 78.284 50.736) (end 78.284 55.308) (width 0.25) (layer F.Cu) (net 15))
 (segment (start 78.284 55.308) (end 77.268 56.324) (width 0.25) (layer F.Cu) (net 15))
 (segment (start 66.35 27) (end 67.502 27) (width 0.25) (layer F.Cu) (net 16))
 (segment (start 67.502 27) (end 68.067 27.565) (width 0.25) (layer F.Cu) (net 16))
 (segment (start 68.067 27.565) (end 69.306 27.565) (width 0.25) (layer F.Cu) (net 16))
 (segment (start 69.306 27.565) (end 69.306 29.312) (width 0.25) (layer F.Cu) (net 16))
 (segment (start 69.306 29.312) (end 70.156 30.162) (width 0.25) (layer F.Cu) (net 16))
 (segment (start 70.156 30.162) (end 74.474 30.162) (width 0.25) (layer F.Cu) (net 16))
 (segment (start 74.474 30.162) (end 74.982 30.67) (width 0.25) (layer F.Cu) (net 16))
 (segment (start 74.982 30.67) (end 74.982 32.194) (width 0.25) (layer F.Cu) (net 16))
 (segment (start 74.982 32.194) (end 73.712 33.464) (width 0.25) (layer F.Cu) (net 16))
 (segment (start 73.712 33.464) (end 71.934 33.464) (width 0.25) (layer F.Cu) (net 16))
 (segment (start 71.934 33.464) (end 71.426 33.972) (width 0.25) (layer F.Cu) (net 16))
 (segment (start 71.426 33.972) (end 71.426 39.052) (width 0.25) (layer F.Cu) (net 16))
 (segment (start 71.426 39.052) (end 74.982 42.608) (width 0.25) (layer F.Cu) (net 16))
 (segment (start 74.982 42.608) (end 74.982 45.402) (width 0.25) (layer F.Cu) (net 16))
 (segment (start 74.982 45.402) (end 77.014 47.434) (width 0.25) (layer F.Cu) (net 16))
 (segment (start 65.1169 19.7865) (end 64.1169 18.7865) (width 0.25) (layer B.Cu) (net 17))
 (segment (start 64.1169 18.7865) (end 64.1169 17.0865) (width 0.25) (layer B.Cu) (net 17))
 (segment (start 70.1169 19.7865) (end 65.1169 19.7865) (width 0.25) (layer B.Cu) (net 17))
 (segment (start 71.1169 17.0865) (end 71.1169 18.7865) (width 0.25) (layer B.Cu) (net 17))
 (segment (start 71.1169 18.7865) (end 70.1169 19.7865) (width 0.25) (layer B.Cu) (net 17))
 (segment (start 71.6648 60.9912) (end 72.188 60.468) (width 0.25) (layer F.Cu) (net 19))
 (segment (start 72.188 60.468) (end 69.648 60.468) (width 0.25) (layer F.Cu) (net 19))
 (segment (start 69.648 60.468) (end 69.648 62.2472) (width 0.25) (layer F.Cu) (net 19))
 (segment (start 69.648 62.2472) (end 70.852 63.4512) (width 0.25) (layer F.Cu) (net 19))
 (segment (start 69.2 82.175) (end 70.213 82.175) (width 0.25) (layer F.Cu) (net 20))
 (segment (start 70.213 82.175) (end 72.15 80.238) (width 0.25) (layer F.Cu) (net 20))
 (segment (start 72.15 80.238) (end 72.15 80) (width 0.25) (layer F.Cu) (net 20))
 (segment (start 72.947 72.323) (end 73 72.27) (width 0.25) (layer F.Cu) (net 21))
 (segment (start 69.2 81.525) (end 69.2 76.07) (width 0.25) (layer F.Cu) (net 21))
 (segment (start 69.2 76.07) (end 72.947 72.323) (width 0.25) (layer F.Cu) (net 21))
 (segment (start 72.947 72.323) (end 72.947 71.053) (width 0.25) (layer F.Cu) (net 21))
 (segment (start 72.947 71.053) (end 73 71) (width 0.25) (layer F.Cu) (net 21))
 (segment (start 74.494 28.13) (end 74.494 27.368) (width 0.25) (layer F.Cu) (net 4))
 (segment (start 74.462 35) (end 76.252 33.21) (width 0.762) (layer F.Cu) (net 4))
 (segment (start 76.252 33.21) (end 76.252 29.888) (width 0.762) (layer F.Cu) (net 4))
 (segment (start 76.252 29.888) (end 74.494 28.13) (width 0.762) (layer F.Cu) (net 4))
 (segment (start 74.494 28.13) (end 74.113 27.749) (width 0.762) (layer F.Cu) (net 4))
 (segment (start 73 35) (end 74.462 35) (width 0.762) (layer F.Cu) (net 4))
 (segment (start 73 35) (end 74.462 35) (width 0.762) (layer F.Cu) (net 4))
 (segment (start 71.506 25.665) (end 71.506 25.764) (width 0.25) (layer F.Cu) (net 4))
 (segment (start 63.65 27) (end 62.93 27) (width 0.25) (layer F.Cu) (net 4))
 (segment (start 71.506 25.665) (end 71.351 25.665) (width 0.25) (layer F.Cu) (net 4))
 (segment (start 71.351 25.665) (end 70.41 26.606) (width 0.25) (layer F.Cu) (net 4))
 (segment (start 70.41 26.606) (end 70.41 28.638) (width 0.25) (layer F.Cu) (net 4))
 (segment (start 70.41 28.638) (end 70.664 28.892) (width 0.25) (layer F.Cu) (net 4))
 (segment (start 70.664 28.892) (end 72.97 28.892) (width 0.25) (layer F.Cu) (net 4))
 (segment (start 72.97 28.892) (end 74.113 27.749) (width 0.25) (layer F.Cu) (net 4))
 (segment (start 74.462 35) (end 74.74 35) (width 0.762) (layer F.Cu) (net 4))
 (segment (start 74.74 35) (end 77.014 37.274) (width 0.762) (layer F.Cu) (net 4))
 (segment (start 77.014 37.274) (end 77.014 44.894) (width 0.762) (layer F.Cu) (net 4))
 (segment (start 77.014 44.894) (end 78.792 44.894) (width 0.762) (layer F.Cu) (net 4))
 (segment (start 78.792 44.894) (end 79.3 45.402) (width 0.762) (layer F.Cu) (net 4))
 (segment (start 79.3 45.402) (end 79.3 64.96) (width 0.762) (layer F.Cu) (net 4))
 (segment (start 79.3 64.96) (end 74.982 69.278) (width 0.762) (layer F.Cu) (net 4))
 (segment (start 73 74.2) (end 73.616 74.2) (width 0.762) (layer F.Cu) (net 4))
 (segment (start 73.616 74.2) (end 74.982 72.834) (width 0.762) (layer F.Cu) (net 4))
 (segment (start 74.982 72.834) (end 74.982 69.278) (width 0.762) (layer F.Cu) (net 4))
 (segment (start 73 74.2) (end 73 75.932) (width 0.762) (layer F.Cu) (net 4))
 (segment (start 73 75.932) (end 74.85 77.782) (width 0.762) (layer F.Cu) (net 4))
 (segment (start 74.85 77.782) (end 74.85 80) (width 0.762) (layer F.Cu) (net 4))
 (segment (start 74.85 80) (end 74.85 86.682) (width 0.762) (layer F.Cu) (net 4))
 (segment (start 74.85 86.682) (end 74.22 87.312) (width 0.762) (layer F.Cu) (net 4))
 (segment (start 74.22 87.312) (end 69.108 87.312) (width 0.762) (layer F.Cu) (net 4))
 (segment (start 64.8 82.825) (end 66.685 82.825) (width 0.25) (layer F.Cu) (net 4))
 (segment (start 66.685 82.825) (end 67.616 83.756) (width 0.25) (layer F.Cu) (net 4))
 (segment (start 67.616 83.756) (end 67.616 85.82) (width 0.25) (layer F.Cu) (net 4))
 (segment (start 67.616 85.82) (end 69.108 87.312) (width 0.25) (layer F.Cu) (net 4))
 (segment (start 68.632 24.32) (end 71.172 24.32) (width 0.25) (layer F.Cu) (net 4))
 (segment (start 71.172 24.32) (end 71.506 24.654) (width 0.25) (layer F.Cu) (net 4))
 (segment (start 71.506 24.654) (end 71.506 25.665) (width 0.25) (layer F.Cu) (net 4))
 (segment (start 63.65 27) (end 63.65 28.482) (width 0.25) (layer F.Cu) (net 4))
 (segment (start 63.65 28.482) (end 64.06 28.892) (width 0.25) (layer F.Cu) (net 4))
 (segment (start 64.06 28.892) (end 66.854 28.892) (width 0.25) (layer F.Cu) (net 4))
 (segment (start 66.854 28.892) (end 68.124 27.622) (width 0.25) (layer B.Cu) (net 4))
 (segment (start 68.124 27.622) (end 68.124 24.828) (width 0.25) (layer B.Cu) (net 4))
 (segment (start 68.124 24.828) (end 68.632 24.32) (width 0.25) (layer B.Cu) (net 4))
 (segment (start 74.982 69.278) (end 65.838 69.278) (width 0.762) (layer F.Cu) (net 4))
 (segment (start 65.838 69.278) (end 64.52 67.96) (width 0.762) (layer F.Cu) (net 4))
 (segment (start 64.52 67.96) (end 63.5 67.96) (width 0.762) (layer F.Cu) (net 4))
 (via (at 66.854 28.892) (size 0.6) (layers F.Cu B.Cu) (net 4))
 (via (at 68.632 24.32) (size 0.6) (layers F.Cu B.Cu) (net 4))
 (segment (start 62.608 32.448) (end 63.806 32.448) (width 0.25) (layer F.Cu) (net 18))
 (segment (start 63.806 32.448) (end 72.352 32.448) (width 0.762) (layer F.Cu) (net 18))
 (segment (start 72.352 32.448) (end 73 31.8) (width 0.762) (layer F.Cu) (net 18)))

